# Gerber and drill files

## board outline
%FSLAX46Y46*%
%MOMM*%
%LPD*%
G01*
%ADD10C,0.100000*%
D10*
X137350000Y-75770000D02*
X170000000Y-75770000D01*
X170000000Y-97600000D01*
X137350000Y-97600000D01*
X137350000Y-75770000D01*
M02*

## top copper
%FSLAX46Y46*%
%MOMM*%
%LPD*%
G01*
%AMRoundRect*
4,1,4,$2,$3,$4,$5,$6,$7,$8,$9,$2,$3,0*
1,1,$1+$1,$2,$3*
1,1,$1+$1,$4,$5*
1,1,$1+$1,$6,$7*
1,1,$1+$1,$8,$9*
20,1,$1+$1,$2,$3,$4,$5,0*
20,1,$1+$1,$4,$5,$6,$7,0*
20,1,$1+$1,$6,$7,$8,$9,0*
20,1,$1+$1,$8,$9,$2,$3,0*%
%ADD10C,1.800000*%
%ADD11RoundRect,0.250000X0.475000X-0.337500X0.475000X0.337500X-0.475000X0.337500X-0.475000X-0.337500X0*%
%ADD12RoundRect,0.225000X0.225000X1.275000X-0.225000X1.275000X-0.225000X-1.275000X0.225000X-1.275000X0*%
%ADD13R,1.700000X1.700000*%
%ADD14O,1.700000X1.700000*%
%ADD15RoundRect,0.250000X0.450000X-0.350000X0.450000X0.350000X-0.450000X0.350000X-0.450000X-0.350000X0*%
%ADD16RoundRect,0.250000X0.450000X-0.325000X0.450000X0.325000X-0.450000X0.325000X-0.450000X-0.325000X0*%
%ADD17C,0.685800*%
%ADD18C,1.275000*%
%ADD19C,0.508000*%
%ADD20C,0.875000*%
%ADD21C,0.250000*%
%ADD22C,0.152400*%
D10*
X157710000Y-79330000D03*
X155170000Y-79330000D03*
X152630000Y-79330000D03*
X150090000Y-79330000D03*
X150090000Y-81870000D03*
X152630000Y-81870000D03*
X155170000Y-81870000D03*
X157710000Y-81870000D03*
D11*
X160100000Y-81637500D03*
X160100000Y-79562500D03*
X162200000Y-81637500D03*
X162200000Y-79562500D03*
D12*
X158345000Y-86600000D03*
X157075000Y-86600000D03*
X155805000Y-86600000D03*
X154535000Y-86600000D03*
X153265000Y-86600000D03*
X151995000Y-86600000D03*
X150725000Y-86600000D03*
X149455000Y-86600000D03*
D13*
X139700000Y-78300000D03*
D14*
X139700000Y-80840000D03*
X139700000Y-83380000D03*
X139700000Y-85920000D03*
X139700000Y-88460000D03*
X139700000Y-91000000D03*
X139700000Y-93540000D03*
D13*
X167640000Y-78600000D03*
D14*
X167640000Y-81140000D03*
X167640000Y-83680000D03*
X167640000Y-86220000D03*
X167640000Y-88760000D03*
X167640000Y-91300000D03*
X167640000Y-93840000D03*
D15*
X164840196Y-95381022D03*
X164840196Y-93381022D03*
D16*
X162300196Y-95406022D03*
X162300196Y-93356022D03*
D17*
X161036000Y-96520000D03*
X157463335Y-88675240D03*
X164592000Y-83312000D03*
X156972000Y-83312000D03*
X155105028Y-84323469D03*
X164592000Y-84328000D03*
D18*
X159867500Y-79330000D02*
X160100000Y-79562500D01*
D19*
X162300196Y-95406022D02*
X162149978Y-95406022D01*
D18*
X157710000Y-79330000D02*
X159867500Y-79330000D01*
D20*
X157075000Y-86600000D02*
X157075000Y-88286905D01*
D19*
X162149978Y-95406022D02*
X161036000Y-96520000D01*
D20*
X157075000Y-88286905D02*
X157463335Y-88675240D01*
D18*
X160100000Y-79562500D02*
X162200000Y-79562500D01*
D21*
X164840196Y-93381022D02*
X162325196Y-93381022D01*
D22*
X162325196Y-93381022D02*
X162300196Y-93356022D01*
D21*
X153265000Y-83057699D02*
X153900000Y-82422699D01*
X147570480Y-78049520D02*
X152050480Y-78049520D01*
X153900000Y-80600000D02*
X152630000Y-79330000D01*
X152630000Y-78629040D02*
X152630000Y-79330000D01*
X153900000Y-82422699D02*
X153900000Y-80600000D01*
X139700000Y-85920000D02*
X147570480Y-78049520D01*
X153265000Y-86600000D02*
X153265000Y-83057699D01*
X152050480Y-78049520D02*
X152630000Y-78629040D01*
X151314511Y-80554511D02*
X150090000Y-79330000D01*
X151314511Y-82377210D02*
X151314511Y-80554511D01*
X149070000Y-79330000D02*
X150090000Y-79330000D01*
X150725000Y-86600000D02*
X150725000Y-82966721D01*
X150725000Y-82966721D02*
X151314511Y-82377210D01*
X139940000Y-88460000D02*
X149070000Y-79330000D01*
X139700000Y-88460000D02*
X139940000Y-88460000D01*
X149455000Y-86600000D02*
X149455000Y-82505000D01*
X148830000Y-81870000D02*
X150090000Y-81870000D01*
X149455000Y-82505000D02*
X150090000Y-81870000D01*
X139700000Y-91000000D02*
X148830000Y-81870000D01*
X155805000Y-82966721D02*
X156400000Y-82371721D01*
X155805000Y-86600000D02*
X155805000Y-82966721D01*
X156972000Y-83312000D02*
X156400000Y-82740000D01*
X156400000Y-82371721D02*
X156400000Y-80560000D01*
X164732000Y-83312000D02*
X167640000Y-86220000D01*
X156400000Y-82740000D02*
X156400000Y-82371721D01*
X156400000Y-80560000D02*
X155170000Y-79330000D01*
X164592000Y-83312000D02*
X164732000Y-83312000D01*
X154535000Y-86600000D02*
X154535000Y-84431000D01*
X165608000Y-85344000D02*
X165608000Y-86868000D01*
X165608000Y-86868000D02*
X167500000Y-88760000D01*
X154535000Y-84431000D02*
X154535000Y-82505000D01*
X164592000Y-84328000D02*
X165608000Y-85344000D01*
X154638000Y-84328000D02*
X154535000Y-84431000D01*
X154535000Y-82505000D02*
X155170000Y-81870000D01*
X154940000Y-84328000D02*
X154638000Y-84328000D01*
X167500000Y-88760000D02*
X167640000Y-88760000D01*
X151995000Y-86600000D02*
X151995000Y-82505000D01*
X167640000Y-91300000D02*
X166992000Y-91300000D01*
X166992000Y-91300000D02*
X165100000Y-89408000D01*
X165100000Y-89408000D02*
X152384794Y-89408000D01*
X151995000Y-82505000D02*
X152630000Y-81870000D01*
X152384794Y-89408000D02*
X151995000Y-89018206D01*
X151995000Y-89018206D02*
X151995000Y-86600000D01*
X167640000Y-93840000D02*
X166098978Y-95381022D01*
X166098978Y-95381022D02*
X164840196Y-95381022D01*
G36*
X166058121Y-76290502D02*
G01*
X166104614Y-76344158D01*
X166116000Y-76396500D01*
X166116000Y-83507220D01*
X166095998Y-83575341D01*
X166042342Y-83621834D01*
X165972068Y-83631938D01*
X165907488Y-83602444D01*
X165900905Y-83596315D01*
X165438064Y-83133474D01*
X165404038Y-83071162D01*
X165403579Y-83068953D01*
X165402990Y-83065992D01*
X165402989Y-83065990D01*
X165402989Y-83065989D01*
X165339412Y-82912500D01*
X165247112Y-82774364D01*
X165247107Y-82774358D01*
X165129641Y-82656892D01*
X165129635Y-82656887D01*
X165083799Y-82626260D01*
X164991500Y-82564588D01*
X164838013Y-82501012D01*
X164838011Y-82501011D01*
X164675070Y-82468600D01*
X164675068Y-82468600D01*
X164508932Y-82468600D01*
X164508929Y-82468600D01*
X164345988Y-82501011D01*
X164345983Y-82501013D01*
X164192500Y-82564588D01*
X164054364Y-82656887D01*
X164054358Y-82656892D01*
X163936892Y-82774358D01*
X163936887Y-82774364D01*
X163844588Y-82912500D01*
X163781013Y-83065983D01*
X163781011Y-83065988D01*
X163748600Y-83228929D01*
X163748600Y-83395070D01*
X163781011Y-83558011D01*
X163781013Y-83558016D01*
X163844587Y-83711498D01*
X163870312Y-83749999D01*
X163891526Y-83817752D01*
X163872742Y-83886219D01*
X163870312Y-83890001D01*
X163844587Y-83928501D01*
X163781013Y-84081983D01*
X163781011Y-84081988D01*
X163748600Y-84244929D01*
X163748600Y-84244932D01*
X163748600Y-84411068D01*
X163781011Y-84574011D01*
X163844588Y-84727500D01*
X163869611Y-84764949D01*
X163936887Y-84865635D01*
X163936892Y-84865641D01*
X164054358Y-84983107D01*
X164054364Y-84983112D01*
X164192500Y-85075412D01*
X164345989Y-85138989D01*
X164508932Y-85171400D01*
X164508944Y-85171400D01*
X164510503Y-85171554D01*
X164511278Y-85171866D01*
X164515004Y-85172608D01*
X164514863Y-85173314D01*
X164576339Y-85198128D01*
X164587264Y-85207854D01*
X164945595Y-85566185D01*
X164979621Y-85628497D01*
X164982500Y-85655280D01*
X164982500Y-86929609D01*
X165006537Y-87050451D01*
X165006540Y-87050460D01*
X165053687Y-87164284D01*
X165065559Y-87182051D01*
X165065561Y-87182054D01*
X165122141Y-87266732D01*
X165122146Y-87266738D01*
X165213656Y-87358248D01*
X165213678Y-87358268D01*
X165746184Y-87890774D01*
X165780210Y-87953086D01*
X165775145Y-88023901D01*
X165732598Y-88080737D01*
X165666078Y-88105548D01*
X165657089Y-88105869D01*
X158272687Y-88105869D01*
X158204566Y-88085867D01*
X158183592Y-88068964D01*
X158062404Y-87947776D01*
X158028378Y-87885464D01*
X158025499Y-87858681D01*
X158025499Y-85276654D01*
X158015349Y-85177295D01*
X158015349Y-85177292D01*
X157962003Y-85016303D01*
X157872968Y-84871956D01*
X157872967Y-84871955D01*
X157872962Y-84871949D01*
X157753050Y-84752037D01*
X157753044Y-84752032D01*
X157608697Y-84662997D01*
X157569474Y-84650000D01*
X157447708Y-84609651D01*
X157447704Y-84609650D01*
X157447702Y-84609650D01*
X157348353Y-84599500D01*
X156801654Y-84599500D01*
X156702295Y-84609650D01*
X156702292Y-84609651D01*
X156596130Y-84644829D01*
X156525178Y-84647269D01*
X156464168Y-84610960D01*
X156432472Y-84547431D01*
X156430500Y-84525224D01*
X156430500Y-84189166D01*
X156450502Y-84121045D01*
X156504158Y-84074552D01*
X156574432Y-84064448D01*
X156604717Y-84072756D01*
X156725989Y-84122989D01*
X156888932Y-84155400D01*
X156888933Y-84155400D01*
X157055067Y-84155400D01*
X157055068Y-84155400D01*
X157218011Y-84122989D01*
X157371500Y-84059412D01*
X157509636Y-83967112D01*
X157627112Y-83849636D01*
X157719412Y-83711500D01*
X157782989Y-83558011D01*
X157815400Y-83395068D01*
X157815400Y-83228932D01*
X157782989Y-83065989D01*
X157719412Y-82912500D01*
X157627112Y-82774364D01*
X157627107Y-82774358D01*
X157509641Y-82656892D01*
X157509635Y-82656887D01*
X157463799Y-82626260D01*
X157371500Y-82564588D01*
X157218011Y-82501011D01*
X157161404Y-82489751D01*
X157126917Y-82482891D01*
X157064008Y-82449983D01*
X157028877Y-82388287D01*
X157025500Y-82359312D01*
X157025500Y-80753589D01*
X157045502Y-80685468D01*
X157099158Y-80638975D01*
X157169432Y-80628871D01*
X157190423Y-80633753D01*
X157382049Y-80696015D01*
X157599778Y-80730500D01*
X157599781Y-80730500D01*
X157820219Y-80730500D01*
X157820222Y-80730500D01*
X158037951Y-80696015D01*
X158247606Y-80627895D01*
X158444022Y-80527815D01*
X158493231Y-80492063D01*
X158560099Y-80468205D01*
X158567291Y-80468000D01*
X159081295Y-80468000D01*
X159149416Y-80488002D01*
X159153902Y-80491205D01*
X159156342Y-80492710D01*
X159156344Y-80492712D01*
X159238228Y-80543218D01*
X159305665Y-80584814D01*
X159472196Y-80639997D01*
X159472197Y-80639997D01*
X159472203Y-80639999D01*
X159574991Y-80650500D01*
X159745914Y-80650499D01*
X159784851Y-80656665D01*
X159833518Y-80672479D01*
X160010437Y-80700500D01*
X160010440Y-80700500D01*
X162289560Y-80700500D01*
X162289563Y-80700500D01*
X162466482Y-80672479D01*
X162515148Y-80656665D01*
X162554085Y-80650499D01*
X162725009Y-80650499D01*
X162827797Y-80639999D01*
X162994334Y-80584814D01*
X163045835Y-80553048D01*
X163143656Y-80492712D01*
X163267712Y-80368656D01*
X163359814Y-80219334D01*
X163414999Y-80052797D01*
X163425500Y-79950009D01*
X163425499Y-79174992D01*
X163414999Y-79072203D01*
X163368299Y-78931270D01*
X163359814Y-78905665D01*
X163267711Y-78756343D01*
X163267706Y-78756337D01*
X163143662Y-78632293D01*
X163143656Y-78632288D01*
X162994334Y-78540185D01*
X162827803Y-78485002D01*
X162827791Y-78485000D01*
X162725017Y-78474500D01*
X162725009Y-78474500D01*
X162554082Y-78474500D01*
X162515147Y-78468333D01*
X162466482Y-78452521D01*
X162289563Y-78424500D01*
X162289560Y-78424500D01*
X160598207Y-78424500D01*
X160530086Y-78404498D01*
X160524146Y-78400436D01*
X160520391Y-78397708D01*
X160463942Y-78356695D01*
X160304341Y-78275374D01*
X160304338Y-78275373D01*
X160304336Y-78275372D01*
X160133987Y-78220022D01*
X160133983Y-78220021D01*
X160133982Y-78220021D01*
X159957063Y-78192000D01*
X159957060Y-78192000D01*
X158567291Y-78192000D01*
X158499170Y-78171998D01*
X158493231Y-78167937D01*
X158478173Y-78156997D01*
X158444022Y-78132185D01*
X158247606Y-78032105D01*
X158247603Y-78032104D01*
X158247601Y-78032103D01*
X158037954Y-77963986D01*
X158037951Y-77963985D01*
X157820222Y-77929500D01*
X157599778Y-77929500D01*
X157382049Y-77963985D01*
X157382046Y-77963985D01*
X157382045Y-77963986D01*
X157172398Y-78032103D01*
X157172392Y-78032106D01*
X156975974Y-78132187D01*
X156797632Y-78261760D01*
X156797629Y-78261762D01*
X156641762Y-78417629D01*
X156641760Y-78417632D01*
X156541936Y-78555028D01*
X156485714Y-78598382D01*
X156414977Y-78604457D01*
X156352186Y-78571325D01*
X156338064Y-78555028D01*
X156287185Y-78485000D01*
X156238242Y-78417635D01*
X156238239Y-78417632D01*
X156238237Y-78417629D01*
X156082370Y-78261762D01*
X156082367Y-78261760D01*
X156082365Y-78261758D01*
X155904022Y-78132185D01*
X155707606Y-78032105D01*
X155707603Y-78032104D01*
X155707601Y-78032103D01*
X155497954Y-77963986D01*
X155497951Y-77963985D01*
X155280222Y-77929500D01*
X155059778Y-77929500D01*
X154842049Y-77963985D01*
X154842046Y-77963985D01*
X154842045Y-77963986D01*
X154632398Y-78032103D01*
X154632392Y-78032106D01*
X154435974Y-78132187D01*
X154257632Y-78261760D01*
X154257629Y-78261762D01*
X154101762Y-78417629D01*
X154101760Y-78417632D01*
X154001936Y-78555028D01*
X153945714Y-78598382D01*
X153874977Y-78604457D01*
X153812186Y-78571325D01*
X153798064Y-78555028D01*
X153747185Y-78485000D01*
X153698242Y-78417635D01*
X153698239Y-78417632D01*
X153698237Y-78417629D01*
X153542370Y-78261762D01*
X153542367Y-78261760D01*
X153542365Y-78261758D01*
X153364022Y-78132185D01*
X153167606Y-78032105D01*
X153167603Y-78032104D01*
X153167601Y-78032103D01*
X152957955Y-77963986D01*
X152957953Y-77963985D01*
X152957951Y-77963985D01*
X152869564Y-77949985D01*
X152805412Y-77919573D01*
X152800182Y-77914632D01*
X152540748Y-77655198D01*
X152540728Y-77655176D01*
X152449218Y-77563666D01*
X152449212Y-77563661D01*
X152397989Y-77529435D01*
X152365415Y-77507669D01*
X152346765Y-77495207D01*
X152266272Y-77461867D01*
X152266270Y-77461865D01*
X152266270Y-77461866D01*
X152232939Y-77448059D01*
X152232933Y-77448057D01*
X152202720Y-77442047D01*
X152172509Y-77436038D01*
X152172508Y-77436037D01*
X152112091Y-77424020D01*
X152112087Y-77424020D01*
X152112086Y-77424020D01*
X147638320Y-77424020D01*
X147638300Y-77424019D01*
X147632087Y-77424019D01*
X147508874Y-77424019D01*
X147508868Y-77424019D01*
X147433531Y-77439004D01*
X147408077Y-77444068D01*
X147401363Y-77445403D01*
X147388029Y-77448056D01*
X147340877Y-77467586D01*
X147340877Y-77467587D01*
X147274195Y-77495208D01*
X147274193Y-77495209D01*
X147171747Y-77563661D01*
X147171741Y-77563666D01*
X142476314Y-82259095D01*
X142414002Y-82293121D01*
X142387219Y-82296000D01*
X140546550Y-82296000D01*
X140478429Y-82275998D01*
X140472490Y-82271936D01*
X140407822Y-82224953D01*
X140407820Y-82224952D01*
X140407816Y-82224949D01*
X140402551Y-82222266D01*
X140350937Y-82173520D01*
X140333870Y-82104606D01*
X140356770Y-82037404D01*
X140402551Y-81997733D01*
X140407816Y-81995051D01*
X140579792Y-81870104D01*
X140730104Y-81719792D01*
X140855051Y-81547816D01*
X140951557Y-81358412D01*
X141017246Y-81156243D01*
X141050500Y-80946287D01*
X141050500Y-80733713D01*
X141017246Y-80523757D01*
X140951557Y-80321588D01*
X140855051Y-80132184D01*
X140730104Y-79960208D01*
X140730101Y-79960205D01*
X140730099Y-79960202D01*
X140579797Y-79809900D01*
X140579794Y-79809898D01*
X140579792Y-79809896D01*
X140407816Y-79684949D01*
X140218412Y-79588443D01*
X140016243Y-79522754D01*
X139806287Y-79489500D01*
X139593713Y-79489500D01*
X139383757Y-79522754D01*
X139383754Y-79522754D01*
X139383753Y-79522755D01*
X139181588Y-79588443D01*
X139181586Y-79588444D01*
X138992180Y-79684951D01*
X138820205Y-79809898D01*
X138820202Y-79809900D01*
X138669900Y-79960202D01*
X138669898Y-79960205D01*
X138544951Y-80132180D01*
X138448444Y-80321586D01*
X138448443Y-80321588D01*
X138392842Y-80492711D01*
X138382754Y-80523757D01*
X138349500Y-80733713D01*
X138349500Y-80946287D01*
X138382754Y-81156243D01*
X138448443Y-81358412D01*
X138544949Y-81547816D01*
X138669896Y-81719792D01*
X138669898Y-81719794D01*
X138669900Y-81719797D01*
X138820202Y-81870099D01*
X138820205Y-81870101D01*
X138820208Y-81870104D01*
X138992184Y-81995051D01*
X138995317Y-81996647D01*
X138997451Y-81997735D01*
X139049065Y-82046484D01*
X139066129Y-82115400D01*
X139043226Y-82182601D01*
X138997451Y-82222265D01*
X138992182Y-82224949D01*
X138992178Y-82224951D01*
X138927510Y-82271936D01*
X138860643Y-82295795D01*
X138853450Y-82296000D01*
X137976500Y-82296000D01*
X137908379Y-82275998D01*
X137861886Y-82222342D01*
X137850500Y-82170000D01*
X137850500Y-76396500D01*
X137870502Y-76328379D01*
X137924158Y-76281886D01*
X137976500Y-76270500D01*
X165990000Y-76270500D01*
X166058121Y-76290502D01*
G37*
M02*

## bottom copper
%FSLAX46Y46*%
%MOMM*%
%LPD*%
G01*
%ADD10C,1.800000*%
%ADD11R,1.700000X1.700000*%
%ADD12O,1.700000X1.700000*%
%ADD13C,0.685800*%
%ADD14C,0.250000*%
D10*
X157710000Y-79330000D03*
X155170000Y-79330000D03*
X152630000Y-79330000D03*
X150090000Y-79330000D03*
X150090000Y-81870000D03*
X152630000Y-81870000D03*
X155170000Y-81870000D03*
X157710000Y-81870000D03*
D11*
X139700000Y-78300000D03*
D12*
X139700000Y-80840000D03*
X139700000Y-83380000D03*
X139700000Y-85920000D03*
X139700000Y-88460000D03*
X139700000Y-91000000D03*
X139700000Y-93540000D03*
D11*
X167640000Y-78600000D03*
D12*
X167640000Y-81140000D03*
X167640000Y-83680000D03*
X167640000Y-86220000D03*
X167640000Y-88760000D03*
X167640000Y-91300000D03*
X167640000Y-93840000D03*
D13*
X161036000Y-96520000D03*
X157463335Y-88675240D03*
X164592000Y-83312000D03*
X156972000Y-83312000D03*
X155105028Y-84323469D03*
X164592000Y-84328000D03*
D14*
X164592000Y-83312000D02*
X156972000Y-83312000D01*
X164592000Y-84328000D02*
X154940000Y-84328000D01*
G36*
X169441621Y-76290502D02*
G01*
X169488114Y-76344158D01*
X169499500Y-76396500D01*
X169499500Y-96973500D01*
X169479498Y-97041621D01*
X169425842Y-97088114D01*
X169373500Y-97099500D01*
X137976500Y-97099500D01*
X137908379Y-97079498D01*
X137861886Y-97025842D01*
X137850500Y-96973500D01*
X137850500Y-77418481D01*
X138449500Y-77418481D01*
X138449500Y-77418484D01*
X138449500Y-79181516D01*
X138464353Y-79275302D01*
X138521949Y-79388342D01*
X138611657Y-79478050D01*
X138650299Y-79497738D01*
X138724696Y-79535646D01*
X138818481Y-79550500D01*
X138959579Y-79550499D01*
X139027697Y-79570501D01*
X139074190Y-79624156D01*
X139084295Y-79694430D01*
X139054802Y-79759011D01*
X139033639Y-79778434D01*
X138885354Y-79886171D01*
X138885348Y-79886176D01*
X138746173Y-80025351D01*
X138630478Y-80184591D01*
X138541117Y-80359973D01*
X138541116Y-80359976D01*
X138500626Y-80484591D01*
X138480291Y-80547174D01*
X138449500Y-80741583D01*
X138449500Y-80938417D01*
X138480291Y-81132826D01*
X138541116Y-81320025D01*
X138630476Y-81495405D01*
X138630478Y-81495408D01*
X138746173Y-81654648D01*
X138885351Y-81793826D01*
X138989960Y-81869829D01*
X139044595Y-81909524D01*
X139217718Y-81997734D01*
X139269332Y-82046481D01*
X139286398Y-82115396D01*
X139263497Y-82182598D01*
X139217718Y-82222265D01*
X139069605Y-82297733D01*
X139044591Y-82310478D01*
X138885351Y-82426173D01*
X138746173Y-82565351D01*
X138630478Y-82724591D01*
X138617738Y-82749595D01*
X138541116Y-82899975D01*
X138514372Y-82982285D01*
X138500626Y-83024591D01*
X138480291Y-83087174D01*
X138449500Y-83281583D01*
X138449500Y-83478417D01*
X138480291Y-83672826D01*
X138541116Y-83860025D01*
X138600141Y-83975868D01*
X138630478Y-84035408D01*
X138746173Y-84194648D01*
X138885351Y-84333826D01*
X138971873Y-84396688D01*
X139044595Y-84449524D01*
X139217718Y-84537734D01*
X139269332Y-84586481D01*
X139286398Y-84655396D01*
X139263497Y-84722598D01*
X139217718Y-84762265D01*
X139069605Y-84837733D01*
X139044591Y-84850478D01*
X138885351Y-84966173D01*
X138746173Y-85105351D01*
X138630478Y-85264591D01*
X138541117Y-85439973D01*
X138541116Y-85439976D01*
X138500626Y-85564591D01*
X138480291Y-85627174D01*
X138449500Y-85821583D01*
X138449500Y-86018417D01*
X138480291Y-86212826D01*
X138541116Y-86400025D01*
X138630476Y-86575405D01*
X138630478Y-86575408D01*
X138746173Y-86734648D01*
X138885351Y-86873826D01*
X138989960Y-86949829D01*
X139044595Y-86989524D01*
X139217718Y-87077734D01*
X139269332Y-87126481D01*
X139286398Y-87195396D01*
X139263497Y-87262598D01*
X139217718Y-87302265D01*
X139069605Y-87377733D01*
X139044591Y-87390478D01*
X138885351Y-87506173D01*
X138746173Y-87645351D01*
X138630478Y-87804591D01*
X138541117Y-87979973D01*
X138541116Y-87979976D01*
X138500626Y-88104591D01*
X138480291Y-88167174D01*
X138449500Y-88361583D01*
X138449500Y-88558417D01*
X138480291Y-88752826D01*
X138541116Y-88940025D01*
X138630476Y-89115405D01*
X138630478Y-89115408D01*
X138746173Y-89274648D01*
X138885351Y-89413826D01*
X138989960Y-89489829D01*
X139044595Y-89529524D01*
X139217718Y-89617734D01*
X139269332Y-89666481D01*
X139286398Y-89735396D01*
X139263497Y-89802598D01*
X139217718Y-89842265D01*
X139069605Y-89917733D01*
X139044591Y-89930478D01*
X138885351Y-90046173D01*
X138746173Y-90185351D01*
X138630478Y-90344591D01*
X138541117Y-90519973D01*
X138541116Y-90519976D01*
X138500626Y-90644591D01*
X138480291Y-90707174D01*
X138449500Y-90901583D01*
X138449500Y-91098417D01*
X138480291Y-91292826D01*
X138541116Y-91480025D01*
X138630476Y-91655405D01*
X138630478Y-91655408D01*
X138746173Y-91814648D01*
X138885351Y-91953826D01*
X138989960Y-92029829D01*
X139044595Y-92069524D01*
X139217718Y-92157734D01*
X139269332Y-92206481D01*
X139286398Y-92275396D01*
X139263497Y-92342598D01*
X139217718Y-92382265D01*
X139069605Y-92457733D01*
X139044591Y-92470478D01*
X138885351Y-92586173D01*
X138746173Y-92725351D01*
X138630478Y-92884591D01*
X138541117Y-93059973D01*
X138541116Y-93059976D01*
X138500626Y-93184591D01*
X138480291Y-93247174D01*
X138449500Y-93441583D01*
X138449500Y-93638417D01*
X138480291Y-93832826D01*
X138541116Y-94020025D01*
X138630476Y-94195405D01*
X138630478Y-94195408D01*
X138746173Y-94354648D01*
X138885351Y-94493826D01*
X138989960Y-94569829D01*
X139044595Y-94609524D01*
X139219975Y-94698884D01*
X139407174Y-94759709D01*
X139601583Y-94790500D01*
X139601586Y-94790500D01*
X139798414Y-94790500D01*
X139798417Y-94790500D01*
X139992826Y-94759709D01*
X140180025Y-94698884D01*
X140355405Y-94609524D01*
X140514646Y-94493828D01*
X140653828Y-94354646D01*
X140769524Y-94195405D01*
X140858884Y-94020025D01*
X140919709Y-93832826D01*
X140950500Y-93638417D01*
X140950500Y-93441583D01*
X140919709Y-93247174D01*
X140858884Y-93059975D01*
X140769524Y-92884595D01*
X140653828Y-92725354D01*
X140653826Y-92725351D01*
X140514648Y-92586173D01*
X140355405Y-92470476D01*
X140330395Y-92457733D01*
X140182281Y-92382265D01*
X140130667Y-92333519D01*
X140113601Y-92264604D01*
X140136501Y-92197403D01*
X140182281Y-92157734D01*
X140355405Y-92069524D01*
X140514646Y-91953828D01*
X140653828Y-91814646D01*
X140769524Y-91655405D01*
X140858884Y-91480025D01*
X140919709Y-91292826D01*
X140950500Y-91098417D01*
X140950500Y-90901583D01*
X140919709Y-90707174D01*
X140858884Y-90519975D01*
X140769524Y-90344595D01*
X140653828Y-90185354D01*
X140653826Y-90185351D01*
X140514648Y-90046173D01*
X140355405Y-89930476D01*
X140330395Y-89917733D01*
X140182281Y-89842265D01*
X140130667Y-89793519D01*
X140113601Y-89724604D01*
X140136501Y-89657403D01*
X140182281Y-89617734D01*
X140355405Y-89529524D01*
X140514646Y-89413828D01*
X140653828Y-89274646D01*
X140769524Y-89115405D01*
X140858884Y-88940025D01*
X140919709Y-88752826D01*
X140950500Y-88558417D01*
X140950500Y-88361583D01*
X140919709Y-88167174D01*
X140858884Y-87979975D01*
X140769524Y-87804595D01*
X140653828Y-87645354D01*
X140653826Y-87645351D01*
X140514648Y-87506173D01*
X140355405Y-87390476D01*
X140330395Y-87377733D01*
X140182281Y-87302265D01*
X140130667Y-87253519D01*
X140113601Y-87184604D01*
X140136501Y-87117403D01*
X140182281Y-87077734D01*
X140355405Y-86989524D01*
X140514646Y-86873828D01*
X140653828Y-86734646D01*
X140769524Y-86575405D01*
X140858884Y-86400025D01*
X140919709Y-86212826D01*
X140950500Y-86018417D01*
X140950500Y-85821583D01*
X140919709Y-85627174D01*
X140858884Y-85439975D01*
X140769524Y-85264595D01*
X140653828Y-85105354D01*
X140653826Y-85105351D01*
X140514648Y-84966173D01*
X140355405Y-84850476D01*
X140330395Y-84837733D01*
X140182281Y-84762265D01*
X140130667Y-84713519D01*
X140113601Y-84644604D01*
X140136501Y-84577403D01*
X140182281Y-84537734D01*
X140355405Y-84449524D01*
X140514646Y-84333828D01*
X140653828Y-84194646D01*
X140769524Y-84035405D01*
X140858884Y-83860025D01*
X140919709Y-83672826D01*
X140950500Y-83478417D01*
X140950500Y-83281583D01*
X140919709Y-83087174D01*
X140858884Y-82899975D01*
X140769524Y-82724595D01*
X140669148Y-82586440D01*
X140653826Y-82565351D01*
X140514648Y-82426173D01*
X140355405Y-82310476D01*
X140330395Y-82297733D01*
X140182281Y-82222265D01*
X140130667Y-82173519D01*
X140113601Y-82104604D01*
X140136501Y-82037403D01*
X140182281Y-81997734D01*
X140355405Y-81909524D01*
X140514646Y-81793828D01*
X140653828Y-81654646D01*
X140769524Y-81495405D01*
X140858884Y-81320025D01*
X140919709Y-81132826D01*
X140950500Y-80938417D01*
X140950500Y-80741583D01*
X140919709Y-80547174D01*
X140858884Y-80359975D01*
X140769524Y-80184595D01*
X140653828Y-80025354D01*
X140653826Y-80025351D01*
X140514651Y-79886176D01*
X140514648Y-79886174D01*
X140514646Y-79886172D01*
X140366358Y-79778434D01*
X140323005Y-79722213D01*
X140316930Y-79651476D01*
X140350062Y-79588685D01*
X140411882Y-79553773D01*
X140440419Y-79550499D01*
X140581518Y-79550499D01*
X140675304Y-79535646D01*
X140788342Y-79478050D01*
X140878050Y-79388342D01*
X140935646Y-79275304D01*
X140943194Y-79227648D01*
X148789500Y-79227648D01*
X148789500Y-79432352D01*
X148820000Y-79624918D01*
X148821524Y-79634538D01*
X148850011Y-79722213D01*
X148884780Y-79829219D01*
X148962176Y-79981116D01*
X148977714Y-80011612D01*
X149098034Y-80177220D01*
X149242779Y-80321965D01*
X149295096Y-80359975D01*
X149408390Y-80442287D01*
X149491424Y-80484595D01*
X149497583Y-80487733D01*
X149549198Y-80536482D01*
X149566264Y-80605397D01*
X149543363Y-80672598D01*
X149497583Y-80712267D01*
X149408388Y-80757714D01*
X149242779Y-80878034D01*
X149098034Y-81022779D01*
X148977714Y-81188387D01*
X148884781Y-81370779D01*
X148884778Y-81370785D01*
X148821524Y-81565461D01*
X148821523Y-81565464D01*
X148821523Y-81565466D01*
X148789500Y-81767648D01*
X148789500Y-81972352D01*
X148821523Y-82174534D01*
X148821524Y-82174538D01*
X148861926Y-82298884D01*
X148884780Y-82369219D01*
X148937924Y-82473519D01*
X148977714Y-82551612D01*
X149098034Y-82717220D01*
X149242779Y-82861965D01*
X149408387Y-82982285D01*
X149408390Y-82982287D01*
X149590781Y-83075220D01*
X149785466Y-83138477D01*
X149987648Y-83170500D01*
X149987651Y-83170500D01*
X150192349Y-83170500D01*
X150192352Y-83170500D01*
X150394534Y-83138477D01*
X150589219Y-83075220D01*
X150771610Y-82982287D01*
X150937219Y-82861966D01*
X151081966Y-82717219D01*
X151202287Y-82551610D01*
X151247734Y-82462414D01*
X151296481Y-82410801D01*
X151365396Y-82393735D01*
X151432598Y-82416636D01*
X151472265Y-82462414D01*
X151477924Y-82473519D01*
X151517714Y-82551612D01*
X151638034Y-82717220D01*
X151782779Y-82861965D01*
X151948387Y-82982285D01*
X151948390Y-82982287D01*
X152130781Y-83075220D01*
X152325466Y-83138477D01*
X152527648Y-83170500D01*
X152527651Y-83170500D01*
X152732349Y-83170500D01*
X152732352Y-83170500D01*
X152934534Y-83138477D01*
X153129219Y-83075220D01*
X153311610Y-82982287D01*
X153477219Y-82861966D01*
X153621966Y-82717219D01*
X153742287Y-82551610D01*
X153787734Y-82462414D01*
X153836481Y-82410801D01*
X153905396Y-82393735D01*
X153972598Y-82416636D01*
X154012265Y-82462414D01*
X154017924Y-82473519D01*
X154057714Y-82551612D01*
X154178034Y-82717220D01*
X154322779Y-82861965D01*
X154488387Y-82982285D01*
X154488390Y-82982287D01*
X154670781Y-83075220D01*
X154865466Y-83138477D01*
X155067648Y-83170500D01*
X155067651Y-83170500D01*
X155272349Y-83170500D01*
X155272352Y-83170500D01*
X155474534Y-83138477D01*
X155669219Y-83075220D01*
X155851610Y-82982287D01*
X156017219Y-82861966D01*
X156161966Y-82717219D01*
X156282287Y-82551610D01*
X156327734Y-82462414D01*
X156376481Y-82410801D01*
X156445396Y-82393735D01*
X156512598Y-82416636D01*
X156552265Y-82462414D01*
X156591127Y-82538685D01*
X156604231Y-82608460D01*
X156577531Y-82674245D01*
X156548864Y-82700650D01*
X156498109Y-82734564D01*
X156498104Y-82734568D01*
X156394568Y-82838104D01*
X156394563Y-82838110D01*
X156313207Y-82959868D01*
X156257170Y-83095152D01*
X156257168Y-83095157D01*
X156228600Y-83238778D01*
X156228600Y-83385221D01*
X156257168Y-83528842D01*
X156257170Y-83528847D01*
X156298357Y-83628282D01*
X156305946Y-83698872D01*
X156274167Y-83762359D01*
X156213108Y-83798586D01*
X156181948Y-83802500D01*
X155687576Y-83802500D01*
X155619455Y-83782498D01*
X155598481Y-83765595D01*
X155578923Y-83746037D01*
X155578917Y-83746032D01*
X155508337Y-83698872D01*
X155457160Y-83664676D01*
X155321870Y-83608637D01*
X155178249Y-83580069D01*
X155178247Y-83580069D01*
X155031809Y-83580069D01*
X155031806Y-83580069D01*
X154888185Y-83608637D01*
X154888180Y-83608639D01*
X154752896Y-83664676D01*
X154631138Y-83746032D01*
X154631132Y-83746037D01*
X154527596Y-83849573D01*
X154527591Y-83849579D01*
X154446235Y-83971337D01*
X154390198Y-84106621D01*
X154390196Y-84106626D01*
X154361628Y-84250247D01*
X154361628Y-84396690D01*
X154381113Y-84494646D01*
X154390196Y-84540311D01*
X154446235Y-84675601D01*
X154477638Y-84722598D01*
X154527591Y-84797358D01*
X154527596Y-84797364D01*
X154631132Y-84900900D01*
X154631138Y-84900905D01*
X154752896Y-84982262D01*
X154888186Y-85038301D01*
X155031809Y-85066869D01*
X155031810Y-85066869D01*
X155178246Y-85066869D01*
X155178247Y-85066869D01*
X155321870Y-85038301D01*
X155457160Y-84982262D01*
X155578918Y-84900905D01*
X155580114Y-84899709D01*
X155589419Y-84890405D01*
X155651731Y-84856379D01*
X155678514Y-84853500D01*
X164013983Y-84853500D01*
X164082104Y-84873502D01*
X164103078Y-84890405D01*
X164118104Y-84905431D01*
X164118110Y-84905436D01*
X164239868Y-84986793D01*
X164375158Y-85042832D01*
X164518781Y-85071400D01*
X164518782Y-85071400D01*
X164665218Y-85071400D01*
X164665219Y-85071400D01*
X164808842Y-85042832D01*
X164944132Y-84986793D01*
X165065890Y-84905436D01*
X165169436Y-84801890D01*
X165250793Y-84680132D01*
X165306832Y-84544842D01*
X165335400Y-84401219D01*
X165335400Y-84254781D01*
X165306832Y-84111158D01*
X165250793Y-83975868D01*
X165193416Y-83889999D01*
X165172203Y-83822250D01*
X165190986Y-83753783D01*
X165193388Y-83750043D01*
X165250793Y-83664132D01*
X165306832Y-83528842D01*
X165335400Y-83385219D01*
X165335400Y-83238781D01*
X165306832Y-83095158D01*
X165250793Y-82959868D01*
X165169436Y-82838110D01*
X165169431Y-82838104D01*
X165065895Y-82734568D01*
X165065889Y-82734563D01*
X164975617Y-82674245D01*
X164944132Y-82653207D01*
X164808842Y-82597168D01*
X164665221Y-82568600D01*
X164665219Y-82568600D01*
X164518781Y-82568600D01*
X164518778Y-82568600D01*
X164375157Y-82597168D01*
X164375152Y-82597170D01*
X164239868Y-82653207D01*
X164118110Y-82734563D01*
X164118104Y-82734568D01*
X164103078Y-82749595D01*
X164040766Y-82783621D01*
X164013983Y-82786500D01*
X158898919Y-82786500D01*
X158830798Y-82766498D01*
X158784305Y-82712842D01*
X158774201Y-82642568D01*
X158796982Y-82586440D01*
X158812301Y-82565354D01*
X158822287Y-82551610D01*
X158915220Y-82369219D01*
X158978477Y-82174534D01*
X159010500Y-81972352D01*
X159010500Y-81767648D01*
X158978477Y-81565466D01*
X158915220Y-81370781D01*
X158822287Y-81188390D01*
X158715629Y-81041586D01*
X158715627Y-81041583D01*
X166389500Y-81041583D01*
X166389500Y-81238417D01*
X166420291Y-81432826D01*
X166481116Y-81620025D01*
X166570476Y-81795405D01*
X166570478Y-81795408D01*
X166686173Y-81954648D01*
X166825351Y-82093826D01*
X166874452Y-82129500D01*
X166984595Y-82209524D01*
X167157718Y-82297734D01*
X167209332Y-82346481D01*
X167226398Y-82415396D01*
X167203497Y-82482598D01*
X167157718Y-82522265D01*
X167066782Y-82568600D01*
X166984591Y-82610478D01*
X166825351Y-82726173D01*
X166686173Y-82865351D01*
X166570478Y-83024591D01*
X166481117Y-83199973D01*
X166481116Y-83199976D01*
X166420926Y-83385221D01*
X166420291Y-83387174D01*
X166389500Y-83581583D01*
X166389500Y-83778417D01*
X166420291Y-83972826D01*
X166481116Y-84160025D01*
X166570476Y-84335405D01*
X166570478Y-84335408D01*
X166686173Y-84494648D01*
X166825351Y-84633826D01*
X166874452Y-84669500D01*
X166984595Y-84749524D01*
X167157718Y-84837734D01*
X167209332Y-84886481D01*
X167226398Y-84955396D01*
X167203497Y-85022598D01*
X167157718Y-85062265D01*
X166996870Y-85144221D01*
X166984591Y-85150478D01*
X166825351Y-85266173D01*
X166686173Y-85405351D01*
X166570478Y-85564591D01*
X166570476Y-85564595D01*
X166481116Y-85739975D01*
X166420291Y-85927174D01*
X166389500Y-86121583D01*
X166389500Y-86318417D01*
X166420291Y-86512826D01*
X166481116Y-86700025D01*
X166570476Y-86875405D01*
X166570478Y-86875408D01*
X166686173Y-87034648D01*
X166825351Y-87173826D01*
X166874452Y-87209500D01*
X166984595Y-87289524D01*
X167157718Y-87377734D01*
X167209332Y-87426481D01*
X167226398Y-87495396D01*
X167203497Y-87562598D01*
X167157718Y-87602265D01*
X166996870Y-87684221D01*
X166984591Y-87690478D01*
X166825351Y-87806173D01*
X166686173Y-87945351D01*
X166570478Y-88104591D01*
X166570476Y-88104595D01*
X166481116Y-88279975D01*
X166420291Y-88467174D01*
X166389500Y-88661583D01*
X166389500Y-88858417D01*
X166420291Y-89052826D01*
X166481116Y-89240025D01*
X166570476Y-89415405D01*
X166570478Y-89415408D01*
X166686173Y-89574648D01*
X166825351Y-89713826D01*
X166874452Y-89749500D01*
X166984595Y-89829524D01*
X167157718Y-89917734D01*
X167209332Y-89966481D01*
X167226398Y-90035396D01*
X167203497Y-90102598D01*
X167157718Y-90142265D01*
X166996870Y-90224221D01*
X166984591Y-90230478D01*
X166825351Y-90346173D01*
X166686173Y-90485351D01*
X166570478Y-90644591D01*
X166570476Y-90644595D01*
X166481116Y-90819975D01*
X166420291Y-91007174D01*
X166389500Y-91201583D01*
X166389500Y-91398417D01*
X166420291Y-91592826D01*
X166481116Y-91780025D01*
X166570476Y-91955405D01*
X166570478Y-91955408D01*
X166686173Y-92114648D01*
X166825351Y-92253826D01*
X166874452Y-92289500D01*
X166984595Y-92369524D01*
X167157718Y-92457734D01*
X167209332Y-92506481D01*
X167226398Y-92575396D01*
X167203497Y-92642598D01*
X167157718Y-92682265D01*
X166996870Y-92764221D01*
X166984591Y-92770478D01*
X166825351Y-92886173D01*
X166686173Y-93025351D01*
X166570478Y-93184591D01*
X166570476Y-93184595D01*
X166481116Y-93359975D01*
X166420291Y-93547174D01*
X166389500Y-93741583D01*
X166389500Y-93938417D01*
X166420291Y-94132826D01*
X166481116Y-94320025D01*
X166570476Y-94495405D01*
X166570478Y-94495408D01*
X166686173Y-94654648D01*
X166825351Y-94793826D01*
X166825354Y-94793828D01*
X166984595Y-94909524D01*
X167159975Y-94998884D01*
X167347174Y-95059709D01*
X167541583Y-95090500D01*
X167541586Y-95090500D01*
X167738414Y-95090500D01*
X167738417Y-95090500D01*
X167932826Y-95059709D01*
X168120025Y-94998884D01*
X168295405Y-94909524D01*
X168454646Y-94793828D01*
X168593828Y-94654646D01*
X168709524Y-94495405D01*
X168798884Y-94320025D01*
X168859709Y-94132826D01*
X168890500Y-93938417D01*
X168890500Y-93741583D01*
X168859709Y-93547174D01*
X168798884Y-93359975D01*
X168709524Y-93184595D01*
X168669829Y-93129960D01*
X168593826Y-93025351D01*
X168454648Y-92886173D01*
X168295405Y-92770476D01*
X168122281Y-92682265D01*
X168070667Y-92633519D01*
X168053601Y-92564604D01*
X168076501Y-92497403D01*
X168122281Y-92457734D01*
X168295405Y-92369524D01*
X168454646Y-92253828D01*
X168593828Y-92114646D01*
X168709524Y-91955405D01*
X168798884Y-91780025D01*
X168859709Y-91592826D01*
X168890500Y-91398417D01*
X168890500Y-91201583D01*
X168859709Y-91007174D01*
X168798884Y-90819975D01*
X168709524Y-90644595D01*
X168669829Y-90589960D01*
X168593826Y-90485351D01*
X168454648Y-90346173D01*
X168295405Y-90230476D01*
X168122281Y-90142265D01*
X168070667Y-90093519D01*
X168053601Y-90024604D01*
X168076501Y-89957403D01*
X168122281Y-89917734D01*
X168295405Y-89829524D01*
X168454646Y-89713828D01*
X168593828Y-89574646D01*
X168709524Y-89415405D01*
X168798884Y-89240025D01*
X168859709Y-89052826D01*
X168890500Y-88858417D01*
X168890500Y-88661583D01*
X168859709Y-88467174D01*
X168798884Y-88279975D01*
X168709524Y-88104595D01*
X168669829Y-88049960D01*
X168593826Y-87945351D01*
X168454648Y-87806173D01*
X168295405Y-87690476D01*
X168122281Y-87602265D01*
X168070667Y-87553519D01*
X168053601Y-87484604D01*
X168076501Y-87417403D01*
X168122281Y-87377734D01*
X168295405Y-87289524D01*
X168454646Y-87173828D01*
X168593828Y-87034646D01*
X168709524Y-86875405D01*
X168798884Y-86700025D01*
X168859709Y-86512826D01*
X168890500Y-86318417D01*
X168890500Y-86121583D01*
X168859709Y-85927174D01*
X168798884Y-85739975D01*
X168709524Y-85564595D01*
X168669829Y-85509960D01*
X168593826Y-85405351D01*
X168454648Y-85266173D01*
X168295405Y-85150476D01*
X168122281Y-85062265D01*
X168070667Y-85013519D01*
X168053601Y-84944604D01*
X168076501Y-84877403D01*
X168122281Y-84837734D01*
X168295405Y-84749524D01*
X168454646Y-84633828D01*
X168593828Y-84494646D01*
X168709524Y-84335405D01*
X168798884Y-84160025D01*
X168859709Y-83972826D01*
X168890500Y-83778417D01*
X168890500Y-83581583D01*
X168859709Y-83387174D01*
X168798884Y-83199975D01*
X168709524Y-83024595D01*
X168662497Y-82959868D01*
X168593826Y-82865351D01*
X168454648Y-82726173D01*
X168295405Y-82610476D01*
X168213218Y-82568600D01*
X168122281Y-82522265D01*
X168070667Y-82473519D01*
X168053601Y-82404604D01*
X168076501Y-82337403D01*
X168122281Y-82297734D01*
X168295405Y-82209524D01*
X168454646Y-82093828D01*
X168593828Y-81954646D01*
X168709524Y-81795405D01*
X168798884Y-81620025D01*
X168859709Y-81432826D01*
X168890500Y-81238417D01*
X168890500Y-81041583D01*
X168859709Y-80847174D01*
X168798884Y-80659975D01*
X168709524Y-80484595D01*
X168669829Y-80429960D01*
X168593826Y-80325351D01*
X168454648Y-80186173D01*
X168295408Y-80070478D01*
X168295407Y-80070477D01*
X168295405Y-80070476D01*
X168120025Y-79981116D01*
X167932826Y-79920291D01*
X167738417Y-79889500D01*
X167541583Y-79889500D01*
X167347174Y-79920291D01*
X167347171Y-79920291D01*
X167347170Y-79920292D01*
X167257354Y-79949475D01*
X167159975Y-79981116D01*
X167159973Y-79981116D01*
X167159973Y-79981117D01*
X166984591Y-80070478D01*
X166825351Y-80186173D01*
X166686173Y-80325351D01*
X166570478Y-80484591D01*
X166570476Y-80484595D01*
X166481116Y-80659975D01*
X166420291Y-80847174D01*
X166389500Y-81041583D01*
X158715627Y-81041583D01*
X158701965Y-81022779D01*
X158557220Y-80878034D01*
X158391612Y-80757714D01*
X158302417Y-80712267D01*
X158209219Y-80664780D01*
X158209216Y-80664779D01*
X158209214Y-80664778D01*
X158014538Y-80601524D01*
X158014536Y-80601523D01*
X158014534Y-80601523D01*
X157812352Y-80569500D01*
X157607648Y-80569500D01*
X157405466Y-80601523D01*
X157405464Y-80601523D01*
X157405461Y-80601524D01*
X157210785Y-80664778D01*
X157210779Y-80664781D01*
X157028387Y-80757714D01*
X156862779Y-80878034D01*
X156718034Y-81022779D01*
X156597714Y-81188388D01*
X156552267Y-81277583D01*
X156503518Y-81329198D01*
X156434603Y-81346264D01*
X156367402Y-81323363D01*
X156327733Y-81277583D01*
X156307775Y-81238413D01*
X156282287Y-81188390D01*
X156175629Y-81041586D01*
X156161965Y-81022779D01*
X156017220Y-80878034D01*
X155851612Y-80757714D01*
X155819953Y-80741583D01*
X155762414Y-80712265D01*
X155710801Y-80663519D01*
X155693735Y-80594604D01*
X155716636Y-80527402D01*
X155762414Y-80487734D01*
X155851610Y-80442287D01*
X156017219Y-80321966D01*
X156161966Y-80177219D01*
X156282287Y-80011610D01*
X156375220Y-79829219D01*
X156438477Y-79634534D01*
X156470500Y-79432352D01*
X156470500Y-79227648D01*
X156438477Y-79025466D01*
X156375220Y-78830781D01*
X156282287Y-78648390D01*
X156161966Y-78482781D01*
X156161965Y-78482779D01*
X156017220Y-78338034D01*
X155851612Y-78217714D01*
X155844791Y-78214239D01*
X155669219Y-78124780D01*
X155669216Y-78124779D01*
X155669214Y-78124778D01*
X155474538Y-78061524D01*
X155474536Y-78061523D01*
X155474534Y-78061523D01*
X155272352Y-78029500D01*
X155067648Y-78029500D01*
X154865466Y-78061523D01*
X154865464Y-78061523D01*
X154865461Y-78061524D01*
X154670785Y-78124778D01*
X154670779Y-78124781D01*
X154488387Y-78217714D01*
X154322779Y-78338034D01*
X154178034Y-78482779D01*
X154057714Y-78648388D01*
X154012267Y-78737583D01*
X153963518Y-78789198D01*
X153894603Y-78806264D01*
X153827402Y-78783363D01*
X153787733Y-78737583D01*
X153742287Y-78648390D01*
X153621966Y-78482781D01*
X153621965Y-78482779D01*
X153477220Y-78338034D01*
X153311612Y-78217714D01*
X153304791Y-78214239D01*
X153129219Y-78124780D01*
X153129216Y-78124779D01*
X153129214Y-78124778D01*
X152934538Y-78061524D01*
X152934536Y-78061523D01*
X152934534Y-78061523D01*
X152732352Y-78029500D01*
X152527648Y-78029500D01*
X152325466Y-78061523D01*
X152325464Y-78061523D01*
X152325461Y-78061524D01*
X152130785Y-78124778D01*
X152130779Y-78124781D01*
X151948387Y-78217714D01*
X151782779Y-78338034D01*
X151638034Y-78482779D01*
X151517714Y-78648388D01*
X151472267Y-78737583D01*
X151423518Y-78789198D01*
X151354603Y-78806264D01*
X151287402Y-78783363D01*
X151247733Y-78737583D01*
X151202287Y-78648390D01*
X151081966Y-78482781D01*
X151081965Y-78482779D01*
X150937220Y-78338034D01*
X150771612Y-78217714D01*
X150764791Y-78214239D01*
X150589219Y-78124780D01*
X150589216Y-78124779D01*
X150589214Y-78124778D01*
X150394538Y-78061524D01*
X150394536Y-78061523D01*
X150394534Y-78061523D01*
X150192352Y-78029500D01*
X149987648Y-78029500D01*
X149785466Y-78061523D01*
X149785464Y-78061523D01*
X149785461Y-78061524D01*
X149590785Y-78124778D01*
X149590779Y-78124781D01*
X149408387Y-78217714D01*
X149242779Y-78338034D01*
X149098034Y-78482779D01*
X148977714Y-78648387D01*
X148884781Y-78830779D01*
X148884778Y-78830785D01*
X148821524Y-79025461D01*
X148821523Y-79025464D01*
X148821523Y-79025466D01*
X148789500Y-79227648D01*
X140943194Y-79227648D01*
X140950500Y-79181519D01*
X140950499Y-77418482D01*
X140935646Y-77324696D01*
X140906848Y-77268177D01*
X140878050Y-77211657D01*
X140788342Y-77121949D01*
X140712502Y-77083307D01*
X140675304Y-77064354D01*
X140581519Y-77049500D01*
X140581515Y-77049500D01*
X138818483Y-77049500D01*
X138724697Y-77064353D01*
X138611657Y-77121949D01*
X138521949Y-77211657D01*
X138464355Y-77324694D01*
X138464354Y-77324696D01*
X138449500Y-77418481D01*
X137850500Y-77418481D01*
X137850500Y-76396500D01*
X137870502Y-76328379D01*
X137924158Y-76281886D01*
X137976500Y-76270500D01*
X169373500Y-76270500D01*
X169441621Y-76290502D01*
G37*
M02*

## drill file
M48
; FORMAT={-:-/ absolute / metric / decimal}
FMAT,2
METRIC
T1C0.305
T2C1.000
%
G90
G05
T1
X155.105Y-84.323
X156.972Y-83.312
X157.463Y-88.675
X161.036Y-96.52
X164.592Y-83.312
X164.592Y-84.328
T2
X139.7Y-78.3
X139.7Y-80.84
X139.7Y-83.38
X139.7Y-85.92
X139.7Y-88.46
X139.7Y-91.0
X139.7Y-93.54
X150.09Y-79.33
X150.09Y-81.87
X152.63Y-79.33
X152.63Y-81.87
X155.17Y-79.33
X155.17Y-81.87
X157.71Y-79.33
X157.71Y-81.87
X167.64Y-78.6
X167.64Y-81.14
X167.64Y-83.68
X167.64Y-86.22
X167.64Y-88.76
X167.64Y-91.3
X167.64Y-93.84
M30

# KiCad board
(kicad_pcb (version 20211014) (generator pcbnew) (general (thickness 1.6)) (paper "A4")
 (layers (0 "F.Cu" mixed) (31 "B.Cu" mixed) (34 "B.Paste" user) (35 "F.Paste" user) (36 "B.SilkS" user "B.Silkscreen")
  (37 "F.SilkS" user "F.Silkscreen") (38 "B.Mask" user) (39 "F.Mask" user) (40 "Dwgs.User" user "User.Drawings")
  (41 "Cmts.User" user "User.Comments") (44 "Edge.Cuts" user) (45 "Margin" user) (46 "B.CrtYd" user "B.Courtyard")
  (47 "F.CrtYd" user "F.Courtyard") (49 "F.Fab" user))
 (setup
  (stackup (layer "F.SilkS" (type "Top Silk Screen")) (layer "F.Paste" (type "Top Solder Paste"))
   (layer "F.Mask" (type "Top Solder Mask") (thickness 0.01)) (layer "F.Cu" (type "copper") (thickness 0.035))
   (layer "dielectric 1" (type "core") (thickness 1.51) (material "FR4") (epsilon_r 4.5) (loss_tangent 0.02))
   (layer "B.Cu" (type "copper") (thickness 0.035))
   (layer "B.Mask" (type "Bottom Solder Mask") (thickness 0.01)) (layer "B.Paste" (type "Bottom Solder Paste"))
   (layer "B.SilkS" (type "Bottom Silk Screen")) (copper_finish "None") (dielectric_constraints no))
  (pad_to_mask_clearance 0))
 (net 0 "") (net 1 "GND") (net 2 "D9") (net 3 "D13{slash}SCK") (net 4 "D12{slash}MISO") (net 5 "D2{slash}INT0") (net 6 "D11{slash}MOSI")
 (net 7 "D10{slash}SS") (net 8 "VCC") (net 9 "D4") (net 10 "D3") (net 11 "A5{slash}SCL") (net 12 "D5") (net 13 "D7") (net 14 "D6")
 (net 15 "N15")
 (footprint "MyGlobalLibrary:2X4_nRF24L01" (layer "F.Cu") (at 153.9 80.6 180)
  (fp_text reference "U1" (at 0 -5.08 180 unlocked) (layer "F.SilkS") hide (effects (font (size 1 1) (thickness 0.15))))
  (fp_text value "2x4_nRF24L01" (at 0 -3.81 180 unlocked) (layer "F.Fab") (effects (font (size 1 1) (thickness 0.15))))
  (pad "1" thru_hole circle (at -3.81 1.27 180) (size 1.8 1.8) (drill 1) (layers *.Cu *.Mask) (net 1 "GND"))
  (pad "2" thru_hole circle (at -1.27 1.27 180) (size 1.8 1.8) (drill 1) (layers *.Cu *.Mask) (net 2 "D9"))
  (pad "3" thru_hole circle (at 1.27 1.27 180) (size 1.8 1.8) (drill 1) (layers *.Cu *.Mask) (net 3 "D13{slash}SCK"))
  (pad "4" thru_hole circle (at 3.81 1.27 180) (size 1.8 1.8) (drill 1) (layers *.Cu *.Mask) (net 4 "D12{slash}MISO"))
  (pad "5" thru_hole circle (at 3.81 -1.27 180) (size 1.8 1.8) (drill 1) (layers *.Cu *.Mask) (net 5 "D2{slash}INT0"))
  (pad "6" thru_hole circle (at 1.27 -1.27 180) (size 1.8 1.8) (drill 1) (layers *.Cu *.Mask) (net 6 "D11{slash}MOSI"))
  (pad "7" thru_hole circle (at -1.27 -1.27 180) (size 1.8 1.8) (drill 1) (layers *.Cu *.Mask) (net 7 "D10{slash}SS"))
  (pad "8" thru_hole circle (at -3.81 -1.27 180) (size 1.8 1.8) (drill 1) (layers *.Cu *.Mask) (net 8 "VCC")))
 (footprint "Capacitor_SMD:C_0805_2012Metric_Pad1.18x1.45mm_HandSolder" (layer "F.Cu") (at 160.1 80.6 90)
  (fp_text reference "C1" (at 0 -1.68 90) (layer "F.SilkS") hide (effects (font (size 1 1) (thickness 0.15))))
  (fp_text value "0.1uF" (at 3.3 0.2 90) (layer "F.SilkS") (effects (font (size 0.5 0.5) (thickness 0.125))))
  (pad "1" smd roundrect (at -1.0375 0 90) (size 1.175 1.45) (layers "F.Cu" "F.Paste" "F.Mask") (roundrect_rratio 0.2127659574)
   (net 8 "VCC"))
  (pad "2" smd roundrect (at 1.0375 0 90) (size 1.175 1.45) (layers "F.Cu" "F.Paste" "F.Mask") (roundrect_rratio 0.2127659574) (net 1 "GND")))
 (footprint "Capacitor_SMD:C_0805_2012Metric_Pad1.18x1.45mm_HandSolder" (layer "F.Cu") (at 162.2 80.6 90)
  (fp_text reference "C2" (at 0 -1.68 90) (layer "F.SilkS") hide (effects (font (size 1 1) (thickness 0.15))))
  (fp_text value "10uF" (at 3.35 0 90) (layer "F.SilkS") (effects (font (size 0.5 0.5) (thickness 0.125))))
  (pad "1" smd roundrect (at -1.0375 0 90) (size 1.175 1.45) (layers "F.Cu" "F.Paste" "F.Mask") (roundrect_rratio 0.2127659574)
   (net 8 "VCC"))
  (pad "2" smd roundrect (at 1.0375 0 90) (size 1.175 1.45) (layers "F.Cu" "F.Paste" "F.Mask") (roundrect_rratio 0.2127659574) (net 1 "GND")))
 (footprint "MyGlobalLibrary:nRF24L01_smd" (layer "F.Cu") (at 153.9 86.6 180)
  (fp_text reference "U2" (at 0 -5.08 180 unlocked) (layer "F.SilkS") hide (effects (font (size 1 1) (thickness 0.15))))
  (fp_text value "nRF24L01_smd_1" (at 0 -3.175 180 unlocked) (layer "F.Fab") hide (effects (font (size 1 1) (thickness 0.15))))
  (pad "1" smd roundrect (at -4.445 0 180) (size 0.9 3) (layers "F.Cu" "F.Paste" "F.Mask") (roundrect_rratio 0.25) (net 8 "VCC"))
  (pad "2" smd roundrect (at -3.175 0 180) (size 0.9 3) (layers "F.Cu" "F.Paste" "F.Mask") (roundrect_rratio 0.25) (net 1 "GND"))
  (pad "3" smd roundrect (at -1.905 0 180) (size 0.9 3) (layers "F.Cu" "F.Paste" "F.Mask") (roundrect_rratio 0.25) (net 2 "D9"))
  (pad "4" smd roundrect (at -0.635 0 180) (size 0.9 3) (layers "F.Cu" "F.Paste" "F.Mask") (roundrect_rratio 0.25) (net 7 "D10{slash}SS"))
  (pad "5" smd roundrect (at 0.635 0 180) (size 0.9 3) (layers "F.Cu" "F.Paste" "F.Mask") (roundrect_rratio 0.25) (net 3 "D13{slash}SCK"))
  (pad "6" smd roundrect (at 1.905 0 180) (size 0.9 3) (layers "F.Cu" "F.Paste" "F.Mask") (roundrect_rratio 0.25) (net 6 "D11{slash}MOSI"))
  (pad "7" smd roundrect (at 3.175 0 180) (size 0.9 3) (layers "F.Cu" "F.Paste" "F.Mask") (roundrect_rratio 0.25) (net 4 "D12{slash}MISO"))
  (pad "8" smd roundrect (at 4.445 0 180) (size 0.9 3) (layers "F.Cu" "F.Paste" "F.Mask") (roundrect_rratio 0.25) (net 5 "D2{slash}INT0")))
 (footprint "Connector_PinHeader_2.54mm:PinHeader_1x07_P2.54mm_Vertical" (layer "F.Cu") (at 139.7 78.3)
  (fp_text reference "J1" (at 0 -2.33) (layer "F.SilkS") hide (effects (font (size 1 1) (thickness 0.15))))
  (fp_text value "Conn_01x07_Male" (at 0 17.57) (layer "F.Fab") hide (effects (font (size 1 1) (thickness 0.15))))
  (pad "1" thru_hole rect (at 0 0) (size 1.7 1.7) (drill 1) (layers *.Cu *.Mask) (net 8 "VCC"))
  (pad "2" thru_hole oval (at 0 2.54) (size 1.7 1.7) (drill 1) (layers *.Cu *.Mask) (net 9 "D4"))
  (pad "3" thru_hole oval (at 0 5.08) (size 1.7 1.7) (drill 1) (layers *.Cu *.Mask) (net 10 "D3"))
  (pad "4" thru_hole oval (at 0 7.62) (size 1.7 1.7) (drill 1) (layers *.Cu *.Mask) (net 3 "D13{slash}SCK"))
  (pad "5" thru_hole oval (at 0 10.16) (size 1.7 1.7) (drill 1) (layers *.Cu *.Mask) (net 4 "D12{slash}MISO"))
  (pad "6" thru_hole oval (at 0 12.7) (size 1.7 1.7) (drill 1) (layers *.Cu *.Mask) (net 5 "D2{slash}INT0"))
  (pad "7" thru_hole oval (at 0 15.24) (size 1.7 1.7) (drill 1) (layers *.Cu *.Mask) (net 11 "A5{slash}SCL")))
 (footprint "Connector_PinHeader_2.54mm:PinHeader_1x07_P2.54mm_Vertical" (layer "F.Cu") (at 167.64 78.6)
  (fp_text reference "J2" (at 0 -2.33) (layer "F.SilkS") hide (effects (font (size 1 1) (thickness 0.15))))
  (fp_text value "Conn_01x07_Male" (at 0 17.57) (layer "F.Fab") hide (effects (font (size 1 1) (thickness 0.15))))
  (pad "1" thru_hole rect (at 0 0) (size 1.7 1.7) (drill 1) (layers *.Cu *.Mask) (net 1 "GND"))
  (pad "2" thru_hole oval (at 0 2.54) (size 1.7 1.7) (drill 1) (layers *.Cu *.Mask) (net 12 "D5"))
  (pad "3" thru_hole oval (at 0 5.08) (size 1.7 1.7) (drill 1) (layers *.Cu *.Mask) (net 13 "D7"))
  (pad "4" thru_hole oval (at 0 7.62) (size 1.7 1.7) (drill 1) (layers *.Cu *.Mask) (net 2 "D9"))
  (pad "5" thru_hole oval (at 0 10.16) (size 1.7 1.7) (drill 1) (layers *.Cu *.Mask) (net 7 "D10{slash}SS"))
  (pad "6" thru_hole oval (at 0 12.7) (size 1.7 1.7) (drill 1) (layers *.Cu *.Mask) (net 6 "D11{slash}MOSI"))
  (pad "7" thru_hole oval (at 0 15.24) (size 1.7 1.7) (drill 1) (layers *.Cu *.Mask) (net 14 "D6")))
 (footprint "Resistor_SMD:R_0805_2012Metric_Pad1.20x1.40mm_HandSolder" (layer "F.Cu") (at 164.840196 94.381022 90)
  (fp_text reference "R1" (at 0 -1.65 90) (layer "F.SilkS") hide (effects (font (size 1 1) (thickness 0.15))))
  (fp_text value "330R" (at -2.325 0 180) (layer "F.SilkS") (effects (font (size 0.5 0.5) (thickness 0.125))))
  (pad "1" smd roundrect (at -1 0 90) (size 1.2 1.4) (layers "F.Cu" "F.Paste" "F.Mask") (roundrect_rratio 0.2083333333) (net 14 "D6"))
  (pad "2" smd roundrect (at 1 0 90) (size 1.2 1.4) (layers "F.Cu" "F.Paste" "F.Mask") (roundrect_rratio 0.2083333333) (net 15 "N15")))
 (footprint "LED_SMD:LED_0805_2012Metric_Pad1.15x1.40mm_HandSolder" (layer "F.Cu") (at 162.300196 94.381022 90)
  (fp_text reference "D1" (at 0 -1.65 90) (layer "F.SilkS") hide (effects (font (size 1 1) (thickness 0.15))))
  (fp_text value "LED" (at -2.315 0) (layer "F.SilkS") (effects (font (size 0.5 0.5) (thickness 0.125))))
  (pad "1" smd roundrect (at -1.025 0 90) (size 1.15 1.4) (layers "F.Cu" "F.Paste" "F.Mask") (roundrect_rratio 0.2173913043) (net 1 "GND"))
  (pad "2" smd roundrect (at 1.025 0 90) (size 1.15 1.4) (layers "F.Cu" "F.Paste" "F.Mask") (roundrect_rratio 0.2173913043) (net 15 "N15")))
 (gr_rect (start 137.35 75.77) (end 170 97.6) (layer "Edge.Cuts") (width 0.1) (fill none))
 (segment (start 159.8675 79.33) (end 160.1 79.5625) (width 1.275) (layer "F.Cu") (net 1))
 (segment (start 162.300196 95.406022) (end 162.149978 95.406022) (width 0.508) (layer "F.Cu") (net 1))
 (segment (start 157.71 79.33) (end 159.8675 79.33) (width 1.275) (layer "F.Cu") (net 1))
 (segment (start 157.075 86.6) (end 157.075 88.286905) (width 0.875) (layer "F.Cu") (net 1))
 (segment (start 162.149978 95.406022) (end 161.036 96.52) (width 0.508) (layer "F.Cu") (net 1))
 (segment (start 157.075 88.286905) (end 157.463335 88.67524) (width 0.875) (layer "F.Cu") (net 1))
 (segment (start 160.1 79.5625) (end 162.2 79.5625) (width 1.275) (layer "F.Cu") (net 1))
 (via (at 161.036 96.52) (size 0.6858) (drill 0.3048) (layers "F.Cu" "B.Cu") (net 1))
 (via (at 157.463335 88.67524) (size 0.6858) (drill 0.3048) (layers "F.Cu" "B.Cu") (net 1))
 (segment (start 164.840196 93.381022) (end 162.325196 93.381022) (width 0.25) (layer "F.Cu") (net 15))
 (segment (start 162.325196 93.381022) (end 162.300196 93.356022) (width 0.1524) (layer "F.Cu") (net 15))
 (segment (start 153.265 83.057699) (end 153.9 82.422699) (width 0.25) (layer "F.Cu") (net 3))
 (segment (start 147.57048 78.04952) (end 152.05048 78.04952) (width 0.25) (layer "F.Cu") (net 3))
 (segment (start 153.9 80.6) (end 152.63 79.33) (width 0.25) (layer "F.Cu") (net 3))
 (segment (start 152.63 78.62904) (end 152.63 79.33) (width 0.25) (layer "F.Cu") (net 3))
 (segment (start 153.9 82.422699) (end 153.9 80.6) (width 0.25) (layer "F.Cu") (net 3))
 (segment (start 139.7 85.92) (end 147.57048 78.04952) (width 0.25) (layer "F.Cu") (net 3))
 (segment (start 153.265 86.6) (end 153.265 83.057699) (width 0.25) (layer "F.Cu") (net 3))
 (segment (start 152.05048 78.04952) (end 152.63 78.62904) (width 0.25) (layer "F.Cu") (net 3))
 (segment (start 151.314511 80.554511) (end 150.09 79.33) (width 0.25) (layer "F.Cu") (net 4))
 (segment (start 151.314511 82.37721) (end 151.314511 80.554511) (width 0.25) (layer "F.Cu") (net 4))
 (segment (start 149.07 79.33) (end 150.09 79.33) (width 0.25) (layer "F.Cu") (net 4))
 (segment (start 150.725 86.6) (end 150.725 82.966721) (width 0.25) (layer "F.Cu") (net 4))
 (segment (start 150.725 82.966721) (end 151.314511 82.37721) (width 0.25) (layer "F.Cu") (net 4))
 (segment (start 139.94 88.46) (end 149.07 79.33) (width 0.25) (layer "F.Cu") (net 4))
 (segment (start 139.7 88.46) (end 139.94 88.46) (width 0.25) (layer "F.Cu") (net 4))
 (segment (start 149.455 86.6) (end 149.455 82.505) (width 0.25) (layer "F.Cu") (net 5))
 (segment (start 148.83 81.87) (end 150.09 81.87) (width 0.25) (layer "F.Cu") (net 5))
 (segment (start 149.455 82.505) (end 150.09 81.87) (width 0.25) (layer "F.Cu") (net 5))
 (segment (start 139.7 91) (end 148.83 81.87) (width 0.25) (layer "F.Cu") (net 5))
 (segment (start 155.805 82.966721) (end 156.4 82.371721) (width 0.25) (layer "F.Cu") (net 2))
 (segment (start 155.805 86.6) (end 155.805 82.966721) (width 0.25) (layer "F.Cu") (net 2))
 (segment (start 156.972 83.312) (end 156.4 82.74) (width 0.25) (layer "F.Cu") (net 2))
 (segment (start 156.4 82.371721) (end 156.4 80.56) (width 0.25) (layer "F.Cu") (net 2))
 (segment (start 164.732 83.312) (end 167.64 86.22) (width 0.25) (layer "F.Cu") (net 2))
 (segment (start 156.4 82.74) (end 156.4 82.371721) (width 0.25) (layer "F.Cu") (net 2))
 (segment (start 156.4 80.56) (end 155.17 79.33) (width 0.25) (layer "F.Cu") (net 2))
 (segment (start 164.592 83.312) (end 164.732 83.312) (width 0.25) (layer "F.Cu") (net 2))
 (via (at 164.592 83.312) (size 0.6858) (drill 0.3048) (layers "F.Cu" "B.Cu") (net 2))
 (via (at 156.972 83.312) (size 0.6858) (drill 0.3048) (layers "F.Cu" "B.Cu") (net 2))
 (segment (start 164.592 83.312) (end 156.972 83.312) (width 0.25) (layer "B.Cu") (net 2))
 (segment (start 154.535 86.6) (end 154.535 84.431) (width 0.25) (layer "F.Cu") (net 7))
 (segment (start 165.608 85.344) (end 165.608 86.868) (width 0.25) (layer "F.Cu") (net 7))
 (segment (start 165.608 86.868) (end 167.5 88.76) (width 0.25) (layer "F.Cu") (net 7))
 (segment (start 154.535 84.431) (end 154.535 82.505) (width 0.25) (layer "F.Cu") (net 7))
 (segment (start 164.592 84.328) (end 165.608 85.344) (width 0.25) (layer "F.Cu") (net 7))
 (segment (start 154.638 84.328) (end 154.535 84.431) (width 0.25) (layer "F.Cu") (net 7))
 (segment (start 154.535 82.505) (end 155.17 81.87) (width 0.25) (layer "F.Cu") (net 7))
 (segment (start 154.94 84.328) (end 154.638 84.328) (width 0.25) (layer "F.Cu") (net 7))
 (segment (start 167.5 88.76) (end 167.64 88.76) (width 0.25) (layer "F.Cu") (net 7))
 (via (at 155.105028 84.323469) (size 0.6858) (drill 0.3048) (layers "F.Cu" "B.Cu") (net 7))
 (via (at 164.592 84.328) (size 0.6858) (drill 0.3048) (layers "F.Cu" "B.Cu") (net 7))
 (segment (start 164.592 84.328) (end 154.94 84.328) (width 0.25) (layer "B.Cu") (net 7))
 (segment (start 151.995 86.6) (end 151.995 82.505) (width 0.25) (layer "F.Cu") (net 6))
 (segment (start 167.64 91.3) (end 166.992 91.3) (width 0.25) (layer "F.Cu") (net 6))
 (segment (start 166.992 91.3) (end 165.1 89.408) (width 0.25) (layer "F.Cu") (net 6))
 (segment (start 165.1 89.408) (end 152.384794 89.408) (width 0.25) (layer "F.Cu") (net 6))
 (segment (start 151.995 82.505) (end 152.63 81.87) (width 0.25) (layer "F.Cu") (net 6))
 (segment (start 152.384794 89.408) (end 151.995 89.018206) (width 0.25) (layer "F.Cu") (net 6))
 (segment (start 151.995 89.018206) (end 151.995 86.6) (width 0.25) (layer "F.Cu") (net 6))
 (segment (start 167.64 93.84) (end 166.098978 95.381022) (width 0.25) (layer "F.Cu") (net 14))
 (segment (start 166.098978 95.381022) (end 164.840196 95.381022) (width 0.25) (layer "F.Cu") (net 14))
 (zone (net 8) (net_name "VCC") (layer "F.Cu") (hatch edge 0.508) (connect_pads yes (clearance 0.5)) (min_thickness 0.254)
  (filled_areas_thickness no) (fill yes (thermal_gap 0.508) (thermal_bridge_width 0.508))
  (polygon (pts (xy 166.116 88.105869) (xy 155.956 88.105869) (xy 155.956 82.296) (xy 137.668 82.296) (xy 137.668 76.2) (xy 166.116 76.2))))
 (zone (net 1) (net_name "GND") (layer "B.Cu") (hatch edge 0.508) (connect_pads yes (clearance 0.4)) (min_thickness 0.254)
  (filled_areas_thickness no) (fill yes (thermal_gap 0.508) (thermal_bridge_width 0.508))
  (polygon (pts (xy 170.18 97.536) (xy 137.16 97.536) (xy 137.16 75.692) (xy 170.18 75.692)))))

